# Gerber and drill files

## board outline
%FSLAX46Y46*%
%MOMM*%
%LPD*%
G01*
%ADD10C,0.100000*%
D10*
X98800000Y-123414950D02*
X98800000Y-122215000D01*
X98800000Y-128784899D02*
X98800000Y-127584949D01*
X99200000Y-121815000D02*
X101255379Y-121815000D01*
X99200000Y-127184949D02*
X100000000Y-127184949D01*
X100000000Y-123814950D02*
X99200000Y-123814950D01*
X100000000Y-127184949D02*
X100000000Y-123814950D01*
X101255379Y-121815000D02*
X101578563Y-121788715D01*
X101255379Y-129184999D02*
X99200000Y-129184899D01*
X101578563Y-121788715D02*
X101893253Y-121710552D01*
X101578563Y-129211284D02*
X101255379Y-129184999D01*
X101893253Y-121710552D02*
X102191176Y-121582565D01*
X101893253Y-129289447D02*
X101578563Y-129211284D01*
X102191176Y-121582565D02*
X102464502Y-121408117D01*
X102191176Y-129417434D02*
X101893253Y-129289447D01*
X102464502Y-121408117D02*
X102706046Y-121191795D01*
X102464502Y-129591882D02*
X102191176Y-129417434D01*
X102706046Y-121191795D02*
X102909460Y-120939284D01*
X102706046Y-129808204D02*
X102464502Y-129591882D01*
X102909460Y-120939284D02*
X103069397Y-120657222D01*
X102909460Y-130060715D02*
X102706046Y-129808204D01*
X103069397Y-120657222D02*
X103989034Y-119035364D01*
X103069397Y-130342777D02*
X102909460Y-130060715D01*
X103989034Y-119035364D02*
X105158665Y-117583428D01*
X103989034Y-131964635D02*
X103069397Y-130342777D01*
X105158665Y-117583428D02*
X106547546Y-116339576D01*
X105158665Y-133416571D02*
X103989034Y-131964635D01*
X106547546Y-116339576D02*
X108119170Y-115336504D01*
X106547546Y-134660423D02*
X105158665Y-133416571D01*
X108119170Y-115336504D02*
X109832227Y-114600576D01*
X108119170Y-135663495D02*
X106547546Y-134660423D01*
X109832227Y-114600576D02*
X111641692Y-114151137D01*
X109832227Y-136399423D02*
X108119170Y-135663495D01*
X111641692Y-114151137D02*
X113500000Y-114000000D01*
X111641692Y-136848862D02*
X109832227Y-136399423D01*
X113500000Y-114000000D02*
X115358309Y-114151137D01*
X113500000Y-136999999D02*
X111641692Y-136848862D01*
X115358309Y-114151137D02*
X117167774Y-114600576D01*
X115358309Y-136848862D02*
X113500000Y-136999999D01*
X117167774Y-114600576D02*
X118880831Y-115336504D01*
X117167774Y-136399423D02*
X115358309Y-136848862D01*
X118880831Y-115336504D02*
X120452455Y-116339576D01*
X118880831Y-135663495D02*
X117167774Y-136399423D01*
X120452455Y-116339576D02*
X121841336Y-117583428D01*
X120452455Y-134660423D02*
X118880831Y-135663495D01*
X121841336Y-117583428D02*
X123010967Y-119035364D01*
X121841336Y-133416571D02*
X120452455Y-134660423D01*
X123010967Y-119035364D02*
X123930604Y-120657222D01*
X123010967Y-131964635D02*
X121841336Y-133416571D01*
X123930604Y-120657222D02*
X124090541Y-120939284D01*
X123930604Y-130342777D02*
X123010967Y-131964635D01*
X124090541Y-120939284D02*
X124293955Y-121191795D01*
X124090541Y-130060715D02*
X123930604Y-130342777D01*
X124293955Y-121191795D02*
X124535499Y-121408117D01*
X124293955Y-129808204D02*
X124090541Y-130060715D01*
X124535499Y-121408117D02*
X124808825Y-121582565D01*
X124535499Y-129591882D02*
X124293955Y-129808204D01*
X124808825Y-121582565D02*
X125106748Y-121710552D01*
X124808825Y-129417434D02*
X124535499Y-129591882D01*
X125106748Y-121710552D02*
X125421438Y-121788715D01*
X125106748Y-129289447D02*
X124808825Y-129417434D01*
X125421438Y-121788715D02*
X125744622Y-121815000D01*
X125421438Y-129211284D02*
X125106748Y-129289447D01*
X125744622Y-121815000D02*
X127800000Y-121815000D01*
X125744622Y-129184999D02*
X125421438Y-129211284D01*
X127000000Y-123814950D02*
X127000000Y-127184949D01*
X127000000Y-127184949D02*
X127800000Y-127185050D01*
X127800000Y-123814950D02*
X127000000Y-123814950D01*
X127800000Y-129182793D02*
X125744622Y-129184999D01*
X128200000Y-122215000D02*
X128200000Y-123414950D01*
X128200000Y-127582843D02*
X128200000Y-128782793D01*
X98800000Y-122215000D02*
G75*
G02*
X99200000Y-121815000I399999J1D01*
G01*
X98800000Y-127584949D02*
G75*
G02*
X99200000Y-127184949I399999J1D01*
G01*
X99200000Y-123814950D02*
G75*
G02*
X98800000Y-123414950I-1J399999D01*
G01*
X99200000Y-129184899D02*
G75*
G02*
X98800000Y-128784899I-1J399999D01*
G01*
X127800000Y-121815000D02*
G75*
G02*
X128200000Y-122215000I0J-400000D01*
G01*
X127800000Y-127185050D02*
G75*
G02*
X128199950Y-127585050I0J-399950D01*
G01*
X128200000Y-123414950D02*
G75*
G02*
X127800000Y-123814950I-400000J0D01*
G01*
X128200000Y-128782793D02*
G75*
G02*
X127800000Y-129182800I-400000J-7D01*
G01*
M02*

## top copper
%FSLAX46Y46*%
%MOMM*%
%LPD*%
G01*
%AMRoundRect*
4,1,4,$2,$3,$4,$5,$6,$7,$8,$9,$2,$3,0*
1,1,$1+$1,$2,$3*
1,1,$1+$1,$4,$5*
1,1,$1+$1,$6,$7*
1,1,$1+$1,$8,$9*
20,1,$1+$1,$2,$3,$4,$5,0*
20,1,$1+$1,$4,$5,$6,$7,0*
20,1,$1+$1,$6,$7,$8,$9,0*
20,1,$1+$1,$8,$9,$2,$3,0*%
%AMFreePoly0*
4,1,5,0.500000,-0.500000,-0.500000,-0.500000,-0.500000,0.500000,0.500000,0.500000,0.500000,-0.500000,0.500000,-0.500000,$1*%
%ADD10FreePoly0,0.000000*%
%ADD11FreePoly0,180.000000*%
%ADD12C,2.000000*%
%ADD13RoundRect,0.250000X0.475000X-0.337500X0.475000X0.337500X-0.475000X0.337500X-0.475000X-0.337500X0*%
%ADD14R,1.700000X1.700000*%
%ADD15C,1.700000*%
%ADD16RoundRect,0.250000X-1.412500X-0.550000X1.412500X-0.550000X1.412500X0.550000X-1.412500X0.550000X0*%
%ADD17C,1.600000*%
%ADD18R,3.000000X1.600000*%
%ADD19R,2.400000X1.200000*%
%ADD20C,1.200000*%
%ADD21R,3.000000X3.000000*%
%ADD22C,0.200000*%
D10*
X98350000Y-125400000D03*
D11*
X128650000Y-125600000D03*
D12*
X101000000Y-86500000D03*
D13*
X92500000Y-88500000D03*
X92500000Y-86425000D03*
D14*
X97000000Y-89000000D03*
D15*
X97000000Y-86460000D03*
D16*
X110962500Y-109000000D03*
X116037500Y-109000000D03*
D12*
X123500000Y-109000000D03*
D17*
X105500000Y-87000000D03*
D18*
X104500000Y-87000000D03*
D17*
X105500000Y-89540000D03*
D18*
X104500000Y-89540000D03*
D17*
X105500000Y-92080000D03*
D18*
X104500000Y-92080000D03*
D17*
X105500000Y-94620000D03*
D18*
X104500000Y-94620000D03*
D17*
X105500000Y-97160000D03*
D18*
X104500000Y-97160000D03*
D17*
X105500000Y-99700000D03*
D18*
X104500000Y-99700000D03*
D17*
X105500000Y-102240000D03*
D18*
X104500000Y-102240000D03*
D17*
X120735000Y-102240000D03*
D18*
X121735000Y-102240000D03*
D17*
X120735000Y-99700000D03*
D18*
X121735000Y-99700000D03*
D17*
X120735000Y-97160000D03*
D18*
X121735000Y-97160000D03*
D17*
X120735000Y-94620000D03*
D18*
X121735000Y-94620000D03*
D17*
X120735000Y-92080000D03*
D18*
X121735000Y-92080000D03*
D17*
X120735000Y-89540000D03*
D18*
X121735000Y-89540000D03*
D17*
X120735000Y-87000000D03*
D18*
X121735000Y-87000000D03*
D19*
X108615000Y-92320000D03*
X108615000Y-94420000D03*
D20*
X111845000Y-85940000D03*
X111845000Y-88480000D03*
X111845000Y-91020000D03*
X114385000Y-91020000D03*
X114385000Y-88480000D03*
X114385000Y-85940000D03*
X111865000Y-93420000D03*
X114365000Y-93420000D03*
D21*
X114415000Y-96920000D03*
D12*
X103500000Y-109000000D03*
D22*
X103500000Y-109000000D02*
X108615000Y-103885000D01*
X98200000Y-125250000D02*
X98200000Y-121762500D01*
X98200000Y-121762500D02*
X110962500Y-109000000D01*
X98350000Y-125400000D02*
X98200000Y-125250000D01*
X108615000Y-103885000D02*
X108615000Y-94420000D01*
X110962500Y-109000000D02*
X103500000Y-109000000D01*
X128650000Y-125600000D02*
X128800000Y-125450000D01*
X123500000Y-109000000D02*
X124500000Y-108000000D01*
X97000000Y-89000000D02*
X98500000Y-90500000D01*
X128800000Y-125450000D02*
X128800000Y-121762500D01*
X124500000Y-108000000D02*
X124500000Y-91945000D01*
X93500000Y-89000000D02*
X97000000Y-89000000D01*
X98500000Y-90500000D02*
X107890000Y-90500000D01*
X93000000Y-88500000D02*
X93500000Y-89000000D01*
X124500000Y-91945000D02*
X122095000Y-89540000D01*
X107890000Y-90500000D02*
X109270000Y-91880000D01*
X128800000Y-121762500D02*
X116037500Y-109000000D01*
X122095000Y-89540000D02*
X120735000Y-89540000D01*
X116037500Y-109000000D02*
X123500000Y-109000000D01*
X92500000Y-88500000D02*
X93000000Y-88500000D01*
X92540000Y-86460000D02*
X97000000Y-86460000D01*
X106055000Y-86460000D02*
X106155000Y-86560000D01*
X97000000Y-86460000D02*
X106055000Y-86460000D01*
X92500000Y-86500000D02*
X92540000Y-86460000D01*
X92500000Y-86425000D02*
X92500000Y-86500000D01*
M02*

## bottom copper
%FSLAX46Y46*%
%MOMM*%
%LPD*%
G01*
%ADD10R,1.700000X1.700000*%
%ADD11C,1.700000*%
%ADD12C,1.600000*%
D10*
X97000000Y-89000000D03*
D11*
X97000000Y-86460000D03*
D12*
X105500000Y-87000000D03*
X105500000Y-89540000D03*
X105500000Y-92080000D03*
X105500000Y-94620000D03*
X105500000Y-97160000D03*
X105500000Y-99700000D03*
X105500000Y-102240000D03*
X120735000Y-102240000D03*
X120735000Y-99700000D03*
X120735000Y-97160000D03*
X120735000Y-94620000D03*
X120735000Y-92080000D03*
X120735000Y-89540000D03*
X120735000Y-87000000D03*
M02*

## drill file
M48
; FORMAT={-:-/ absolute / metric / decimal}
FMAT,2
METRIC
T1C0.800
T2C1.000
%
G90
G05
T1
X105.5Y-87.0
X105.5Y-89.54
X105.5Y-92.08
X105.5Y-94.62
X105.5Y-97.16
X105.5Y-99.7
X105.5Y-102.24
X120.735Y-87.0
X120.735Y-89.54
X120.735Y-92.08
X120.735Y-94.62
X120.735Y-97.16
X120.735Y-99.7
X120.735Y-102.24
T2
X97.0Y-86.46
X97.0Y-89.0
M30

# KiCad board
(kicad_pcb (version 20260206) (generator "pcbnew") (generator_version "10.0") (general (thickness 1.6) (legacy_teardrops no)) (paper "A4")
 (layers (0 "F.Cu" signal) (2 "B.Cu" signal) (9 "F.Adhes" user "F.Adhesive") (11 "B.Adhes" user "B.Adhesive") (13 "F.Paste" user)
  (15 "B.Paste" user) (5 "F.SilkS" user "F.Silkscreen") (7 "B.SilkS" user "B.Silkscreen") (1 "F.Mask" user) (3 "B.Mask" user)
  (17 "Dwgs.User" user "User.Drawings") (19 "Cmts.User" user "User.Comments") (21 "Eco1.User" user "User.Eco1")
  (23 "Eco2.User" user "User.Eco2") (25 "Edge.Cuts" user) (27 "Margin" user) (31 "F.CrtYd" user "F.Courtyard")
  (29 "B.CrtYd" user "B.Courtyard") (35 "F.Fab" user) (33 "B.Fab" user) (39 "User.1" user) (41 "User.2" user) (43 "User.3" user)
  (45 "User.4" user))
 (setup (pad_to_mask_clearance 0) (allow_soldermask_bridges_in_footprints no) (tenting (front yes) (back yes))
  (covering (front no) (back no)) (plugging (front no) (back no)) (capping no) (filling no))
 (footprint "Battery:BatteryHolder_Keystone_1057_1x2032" (layer "F.Cu") (at 113.5 125.5)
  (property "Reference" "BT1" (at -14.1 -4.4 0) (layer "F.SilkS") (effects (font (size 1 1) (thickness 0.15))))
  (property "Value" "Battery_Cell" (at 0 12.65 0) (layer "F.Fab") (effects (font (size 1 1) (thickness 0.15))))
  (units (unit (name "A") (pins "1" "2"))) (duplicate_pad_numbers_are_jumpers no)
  (fp_line (start -14.7 -2.08505) (end -14.7 -3.285) (stroke (width 0.1) (type solid)) (layer "Edge.Cuts"))
  (fp_line (start -14.7 3.284899) (end -14.7 2.084949) (stroke (width 0.1) (type solid)) (layer "Edge.Cuts"))
  (fp_line (start -14.3 -3.685) (end -12.244621 -3.685) (stroke (width 0.1) (type solid)) (layer "Edge.Cuts"))
  (fp_line (start -14.3 1.684949) (end -13.5 1.684949) (stroke (width 0.1) (type solid)) (layer "Edge.Cuts"))
  (fp_line (start -13.5 -1.68505) (end -14.3 -1.68505) (stroke (width 0.1) (type solid)) (layer "Edge.Cuts"))
  (fp_line (start -13.5 1.684949) (end -13.5 -1.68505) (stroke (width 0.1) (type solid)) (layer "Edge.Cuts"))
  (fp_line (start -12.244621 -3.685) (end -11.921437 -3.711285) (stroke (width 0.1) (type solid)) (layer "Edge.Cuts"))
  (fp_line (start -12.244621 3.684999) (end -14.3 3.684899) (stroke (width 0.1) (type solid)) (layer "Edge.Cuts"))
  (fp_line (start -11.921437 -3.711285) (end -11.606747 -3.789448) (stroke (width 0.1) (type solid)) (layer "Edge.Cuts"))
  (fp_line (start -11.921437 3.711284) (end -12.244621 3.684999) (stroke (width 0.1) (type solid)) (layer "Edge.Cuts"))
  (fp_line (start -11.606747 -3.789448) (end -11.308824 -3.917435) (stroke (width 0.1) (type solid)) (layer "Edge.Cuts"))
  (fp_line (start -11.606747 3.789447) (end -11.921437 3.711284) (stroke (width 0.1) (type solid)) (layer "Edge.Cuts"))
  (fp_line (start -11.308824 -3.917435) (end -11.035498 -4.091883) (stroke (width 0.1) (type solid)) (layer "Edge.Cuts"))
  (fp_line (start -11.308824 3.917434) (end -11.606747 3.789447) (stroke (width 0.1) (type solid)) (layer "Edge.Cuts"))
  (fp_line (start -11.035498 -4.091883) (end -10.793954 -4.308205) (stroke (width 0.1) (type solid)) (layer "Edge.Cuts"))
  (fp_line (start -11.035498 4.091882) (end -11.308824 3.917434) (stroke (width 0.1) (type solid)) (layer "Edge.Cuts"))
  (fp_line (start -10.793954 -4.308205) (end -10.59054 -4.560716) (stroke (width 0.1) (type solid)) (layer "Edge.Cuts"))
  (fp_line (start -10.793954 4.308204) (end -11.035498 4.091882) (stroke (width 0.1) (type solid)) (layer "Edge.Cuts"))
  (fp_line (start -10.59054 -4.560716) (end -10.430603 -4.842778) (stroke (width 0.1) (type solid)) (layer "Edge.Cuts"))
  (fp_line (start -10.59054 4.560715) (end -10.793954 4.308204) (stroke (width 0.1) (type solid)) (layer "Edge.Cuts"))
  (fp_line (start -10.430603 -4.842778) (end -9.510966 -6.464636) (stroke (width 0.1) (type solid)) (layer "Edge.Cuts"))
  (fp_line (start -10.430603 4.842777) (end -10.59054 4.560715) (stroke (width 0.1) (type solid)) (layer "Edge.Cuts"))
  (fp_line (start -9.510966 -6.464636) (end -8.341335 -7.916572) (stroke (width 0.1) (type solid)) (layer "Edge.Cuts"))
  (fp_line (start -9.510966 6.464635) (end -10.430603 4.842777) (stroke (width 0.1) (type solid)) (layer "Edge.Cuts"))
  (fp_line (start -8.341335 -7.916572) (end -6.952454 -9.160424) (stroke (width 0.1) (type solid)) (layer "Edge.Cuts"))
  (fp_line (start -8.341335 7.916571) (end -9.510966 6.464635) (stroke (width 0.1) (type solid)) (layer "Edge.Cuts"))
  (fp_line (start -6.952454 -9.160424) (end -5.38083 -10.163496) (stroke (width 0.1) (type solid)) (layer "Edge.Cuts"))
  (fp_line (start -6.952454 9.160423) (end -8.341335 7.916571) (stroke (width 0.1) (type solid)) (layer "Edge.Cuts"))
  (fp_line (start -5.38083 -10.163496) (end -3.667773 -10.899424) (stroke (width 0.1) (type solid)) (layer "Edge.Cuts"))
  (fp_line (start -5.38083 10.163495) (end -6.952454 9.160423) (stroke (width 0.1) (type solid)) (layer "Edge.Cuts"))
  (fp_line (start -3.667773 -10.899424) (end -1.858308 -11.348863) (stroke (width 0.1) (type solid)) (layer "Edge.Cuts"))
  (fp_line (start -3.667773 10.899423) (end -5.38083 10.163495) (stroke (width 0.1) (type solid)) (layer "Edge.Cuts"))
  (fp_line (start -1.858308 -11.348863) (end 0 -11.5) (stroke (width 0.1) (type solid)) (layer "Edge.Cuts"))
  (fp_line (start -1.858308 11.348862) (end -3.667773 10.899423) (stroke (width 0.1) (type solid)) (layer "Edge.Cuts"))
  (fp_line (start 0 -11.5) (end 1.858309 -11.348863) (stroke (width 0.1) (type solid)) (layer "Edge.Cuts"))
  (fp_line (start 0 11.499999) (end -1.858308 11.348862) (stroke (width 0.1) (type solid)) (layer "Edge.Cuts"))
  (fp_line (start 1.858309 -11.348863) (end 3.667774 -10.899424) (stroke (width 0.1) (type solid)) (layer "Edge.Cuts"))
  (fp_line (start 1.858309 11.348862) (end 0 11.499999) (stroke (width 0.1) (type solid)) (layer "Edge.Cuts"))
  (fp_line (start 3.667774 -10.899424) (end 5.380831 -10.163496) (stroke (width 0.1) (type solid)) (layer "Edge.Cuts"))
  (fp_line (start 3.667774 10.899423) (end 1.858309 11.348862) (stroke (width 0.1) (type solid)) (layer "Edge.Cuts"))
  (fp_line (start 5.380831 -10.163496) (end 6.952455 -9.160424) (stroke (width 0.1) (type solid)) (layer "Edge.Cuts"))
  (fp_line (start 5.380831 10.163495) (end 3.667774 10.899423) (stroke (width 0.1) (type solid)) (layer "Edge.Cuts"))
  (fp_line (start 6.952455 -9.160424) (end 8.341336 -7.916572) (stroke (width 0.1) (type solid)) (layer "Edge.Cuts"))
  (fp_line (start 6.952455 9.160423) (end 5.380831 10.163495) (stroke (width 0.1) (type solid)) (layer "Edge.Cuts"))
  (fp_line (start 8.341336 -7.916572) (end 9.510967 -6.464636) (stroke (width 0.1) (type solid)) (layer "Edge.Cuts"))
  (fp_line (start 8.341336 7.916571) (end 6.952455 9.160423) (stroke (width 0.1) (type solid)) (layer "Edge.Cuts"))
  (fp_line (start 9.510967 -6.464636) (end 10.430604 -4.842778) (stroke (width 0.1) (type solid)) (layer "Edge.Cuts"))
  (fp_line (start 9.510967 6.464635) (end 8.341336 7.916571) (stroke (width 0.1) (type solid)) (layer "Edge.Cuts"))
  (fp_line (start 10.430604 -4.842778) (end 10.590541 -4.560716) (stroke (width 0.1) (type solid)) (layer "Edge.Cuts"))
  (fp_line (start 10.430604 4.842777) (end 9.510967 6.464635) (stroke (width 0.1) (type solid)) (layer "Edge.Cuts"))
  (fp_line (start 10.590541 -4.560716) (end 10.793955 -4.308205) (stroke (width 0.1) (type solid)) (layer "Edge.Cuts"))
  (fp_line (start 10.590541 4.560715) (end 10.430604 4.842777) (stroke (width 0.1) (type solid)) (layer "Edge.Cuts"))
  (fp_line (start 10.793955 -4.308205) (end 11.035499 -4.091883) (stroke (width 0.1) (type solid)) (layer "Edge.Cuts"))
  (fp_line (start 10.793955 4.308204) (end 10.590541 4.560715) (stroke (width 0.1) (type solid)) (layer "Edge.Cuts"))
  (fp_line (start 11.035499 -4.091883) (end 11.308825 -3.917435) (stroke (width 0.1) (type solid)) (layer "Edge.Cuts"))
  (fp_line (start 11.035499 4.091882) (end 10.793955 4.308204) (stroke (width 0.1) (type solid)) (layer "Edge.Cuts"))
  (fp_line (start 11.308825 -3.917435) (end 11.606748 -3.789448) (stroke (width 0.1) (type solid)) (layer "Edge.Cuts"))
  (fp_line (start 11.308825 3.917434) (end 11.035499 4.091882) (stroke (width 0.1) (type solid)) (layer "Edge.Cuts"))
  (fp_line (start 11.606748 -3.789448) (end 11.921438 -3.711285) (stroke (width 0.1) (type solid)) (layer "Edge.Cuts"))
  (fp_line (start 11.606748 3.789447) (end 11.308825 3.917434) (stroke (width 0.1) (type solid)) (layer "Edge.Cuts"))
  (fp_line (start 11.921438 -3.711285) (end 12.244622 -3.685) (stroke (width 0.1) (type solid)) (layer "Edge.Cuts"))
  (fp_line (start 11.921438 3.711284) (end 11.606748 3.789447) (stroke (width 0.1) (type solid)) (layer "Edge.Cuts"))
  (fp_line (start 12.244622 -3.685) (end 14.3 -3.685) (stroke (width 0.1) (type solid)) (layer "Edge.Cuts"))
  (fp_line (start 12.244622 3.684999) (end 11.921438 3.711284) (stroke (width 0.1) (type solid)) (layer "Edge.Cuts"))
  (fp_line (start 13.5 -1.68505) (end 13.5 1.684949) (stroke (width 0.1) (type solid)) (layer "Edge.Cuts"))
  (fp_line (start 13.5 1.684949) (end 14.3 1.68505) (stroke (width 0.1) (type solid)) (layer "Edge.Cuts"))
  (fp_line (start 14.3 -1.68505) (end 13.5 -1.68505) (stroke (width 0.1) (type solid)) (layer "Edge.Cuts"))
  (fp_line (start 14.3 3.682793) (end 12.244622 3.684999) (stroke (width 0.1) (type solid)) (layer "Edge.Cuts"))
  (fp_line (start 14.7 -3.285) (end 14.7 -2.08505) (stroke (width 0.1) (type solid)) (layer "Edge.Cuts"))
  (fp_line (start 14.7 2.082843) (end 14.7 3.282793) (stroke (width 0.1) (type solid)) (layer "Edge.Cuts"))
  (fp_arc (start -14.7 -3.285) (mid -14.582843 -3.567843) (end -14.3 -3.685) (stroke (width 0.1) (type solid)) (layer "Edge.Cuts"))
  (fp_arc (start -14.7 2.084949) (mid -14.582843 1.802106) (end -14.3 1.684949) (stroke (width 0.1) (type solid)) (layer "Edge.Cuts"))
  (fp_arc (start -14.3 -1.68505) (mid -14.582843 -1.802207) (end -14.7 -2.08505) (stroke (width 0.1) (type solid)) (layer "Edge.Cuts"))
  (fp_arc (start -14.3 3.684899) (mid -14.582843 3.567742) (end -14.7 3.284899) (stroke (width 0.1) (type solid)) (layer "Edge.Cuts"))
  (fp_arc (start 14.3 -3.685) (mid 14.582843 -3.567843) (end 14.7 -3.285) (stroke (width 0.1) (type solid)) (layer "Edge.Cuts"))
  (fp_arc (start 14.3 1.68505) (mid 14.582843 1.802207) (end 14.7 2.08505) (stroke (width 0.1) (type solid)) (layer "Edge.Cuts"))
  (fp_arc (start 14.7 -2.08505) (mid 14.582843 -1.802207) (end 14.3 -1.68505) (stroke (width 0.1) (type solid)) (layer "Edge.Cuts"))
  (fp_arc (start 14.7 3.282793) (mid 14.582843 3.565636) (end 14.3 3.682793) (stroke (width 0.1) (type solid)) (layer "Edge.Cuts"))
  (pad "1" smd custom (at -15.15 -0.1) (size 1 1) (layers "F.Cu" "F.Mask" "F.Paste") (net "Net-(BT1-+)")
   (options (clearance outline) (anchor rect)) (primitives))
  (pad "2" smd custom (at 15.15 0.1 180) (size 1 1) (layers "F.Cu" "F.Mask" "F.Paste") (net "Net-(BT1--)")
   (options (clearance outline) (anchor rect)) (primitives)))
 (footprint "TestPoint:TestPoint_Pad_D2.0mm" (layer "F.Cu") (at 101 86.5)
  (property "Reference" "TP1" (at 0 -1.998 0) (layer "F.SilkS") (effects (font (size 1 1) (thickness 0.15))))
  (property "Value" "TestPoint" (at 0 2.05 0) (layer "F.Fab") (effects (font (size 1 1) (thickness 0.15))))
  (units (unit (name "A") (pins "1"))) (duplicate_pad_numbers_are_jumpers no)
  (pad "1" smd circle (at 0 0) (size 2 2) (layers "F.Cu" "F.Mask") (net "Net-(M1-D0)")))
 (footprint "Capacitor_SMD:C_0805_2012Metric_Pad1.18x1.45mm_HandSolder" (layer "F.Cu") (at 92.5 87.4625 90)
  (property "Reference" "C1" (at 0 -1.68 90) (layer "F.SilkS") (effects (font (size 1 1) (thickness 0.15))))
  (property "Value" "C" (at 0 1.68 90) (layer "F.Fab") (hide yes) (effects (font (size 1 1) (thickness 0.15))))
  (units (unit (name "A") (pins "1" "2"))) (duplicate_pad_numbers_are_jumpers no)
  (pad "1" smd roundrect (at -1.0375 0 90) (size 1.175 1.45) (layers "F.Cu" "F.Mask" "F.Paste") (roundrect_rratio 0.212766)
   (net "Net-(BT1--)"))
  (pad "2" smd roundrect (at 1.0375 0 90) (size 1.175 1.45) (layers "F.Cu" "F.Mask" "F.Paste") (roundrect_rratio 0.212766)
   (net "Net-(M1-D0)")))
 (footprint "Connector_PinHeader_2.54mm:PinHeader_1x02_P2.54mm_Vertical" (layer "F.Cu") (at 97 89 180)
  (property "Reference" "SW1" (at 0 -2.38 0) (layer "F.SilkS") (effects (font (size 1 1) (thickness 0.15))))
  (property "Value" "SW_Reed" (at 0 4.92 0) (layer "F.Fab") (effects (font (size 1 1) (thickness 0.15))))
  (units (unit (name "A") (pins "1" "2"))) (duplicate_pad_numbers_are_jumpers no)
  (pad "1" thru_hole rect (at 0 0 180) (size 1.7 1.7) (drill 1) (layers "*.Cu" "*.Mask") (remove_unused_layers no) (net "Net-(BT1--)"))
  (pad "2" thru_hole circle (at 0 2.54 180) (size 1.7 1.7) (drill 1) (layers "*.Cu" "*.Mask") (remove_unused_layers no) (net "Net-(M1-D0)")))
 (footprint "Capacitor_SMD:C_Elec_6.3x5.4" (layer "F.Cu") (at 113.5 109)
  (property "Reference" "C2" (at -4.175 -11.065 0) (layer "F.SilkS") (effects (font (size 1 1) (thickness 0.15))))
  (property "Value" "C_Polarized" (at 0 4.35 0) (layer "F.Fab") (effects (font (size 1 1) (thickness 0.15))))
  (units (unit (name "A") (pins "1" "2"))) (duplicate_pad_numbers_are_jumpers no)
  (pad "1" smd roundrect (at -2.5375 0) (size 3.325 1.6) (layers "F.Cu" "F.Mask" "F.Paste") (roundrect_rratio 0.15625) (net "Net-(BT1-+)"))
  (pad "2" smd roundrect (at 2.5375 0) (size 3.325 1.6) (layers "F.Cu" "F.Mask" "F.Paste") (roundrect_rratio 0.15625) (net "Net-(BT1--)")))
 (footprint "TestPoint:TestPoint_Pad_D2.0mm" (layer "F.Cu") (at 123.5 109)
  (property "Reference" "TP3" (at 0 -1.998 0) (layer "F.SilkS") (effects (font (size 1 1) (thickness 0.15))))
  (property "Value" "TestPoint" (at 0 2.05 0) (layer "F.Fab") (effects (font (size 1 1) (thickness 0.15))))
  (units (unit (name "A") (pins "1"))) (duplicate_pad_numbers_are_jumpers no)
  (pad "1" smd circle (at 0 0) (size 2 2) (layers "F.Cu" "F.Mask") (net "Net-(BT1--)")))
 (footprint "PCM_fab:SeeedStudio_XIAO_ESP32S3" (layer "F.Cu") (at 113.115 94.62)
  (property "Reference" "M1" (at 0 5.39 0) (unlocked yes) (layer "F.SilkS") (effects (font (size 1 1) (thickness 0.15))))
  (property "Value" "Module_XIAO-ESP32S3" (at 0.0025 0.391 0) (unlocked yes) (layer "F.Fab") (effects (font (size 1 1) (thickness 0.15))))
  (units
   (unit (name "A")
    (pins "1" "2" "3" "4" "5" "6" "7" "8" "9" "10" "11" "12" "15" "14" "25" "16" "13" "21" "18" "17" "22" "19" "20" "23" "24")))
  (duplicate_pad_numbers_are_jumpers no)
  (pad "1" thru_hole circle (at -7.615 -7.62) (size 1.6 1.6) (drill 0.8) (layers "*.Cu" "*.Mask") (remove_unused_layers no)
   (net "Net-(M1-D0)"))
  (pad "1" smd rect (at -7.615 -7.62) (size 3 1.6) (drill (offset -1 0)) (layers "F.Cu" "F.Mask" "F.Paste") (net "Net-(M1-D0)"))
  (pad "2" thru_hole circle (at -7.615 -5.08) (size 1.6 1.6) (drill 0.8) (layers "*.Cu" "*.Mask") (remove_unused_layers no)
   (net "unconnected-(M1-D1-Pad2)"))
  (pad "2" smd rect (at -7.615 -5.08) (size 3 1.6) (drill (offset -1 0)) (layers "F.Cu" "F.Mask" "F.Paste")
   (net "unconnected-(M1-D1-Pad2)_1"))
  (pad "3" thru_hole circle (at -7.615 -2.54) (size 1.6 1.6) (drill 0.8) (layers "*.Cu" "*.Mask") (remove_unused_layers no)
   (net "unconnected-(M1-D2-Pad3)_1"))
  (pad "3" smd rect (at -7.615 -2.54) (size 3 1.6) (drill (offset -1 0)) (layers "F.Cu" "F.Mask" "F.Paste") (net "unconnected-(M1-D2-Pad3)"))
  (pad "4" thru_hole circle (at -7.615 0) (size 1.6 1.6) (drill 0.8) (layers "*.Cu" "*.Mask") (remove_unused_layers no)
   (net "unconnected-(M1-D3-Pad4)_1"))
  (pad "4" smd rect (at -7.615 0) (size 3 1.6) (drill (offset -1 0)) (layers "F.Cu" "F.Mask" "F.Paste") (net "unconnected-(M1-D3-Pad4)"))
  (pad "5" thru_hole circle (at -7.615 2.54) (size 1.6 1.6) (drill 0.8) (layers "*.Cu" "*.Mask") (remove_unused_layers no)
   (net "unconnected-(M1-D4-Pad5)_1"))
  (pad "5" smd rect (at -7.615 2.54) (size 3 1.6) (drill (offset -1 0)) (layers "F.Cu" "F.Mask" "F.Paste") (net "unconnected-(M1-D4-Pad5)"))
  (pad "6" thru_hole circle (at -7.615 5.08) (size 1.6 1.6) (drill 0.8) (layers "*.Cu" "*.Mask") (remove_unused_layers no)
   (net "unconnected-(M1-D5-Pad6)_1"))
  (pad "6" smd rect (at -7.615 5.08) (size 3 1.6) (drill (offset -1 0)) (layers "F.Cu" "F.Mask" "F.Paste") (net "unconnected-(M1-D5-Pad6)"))
  (pad "7" thru_hole circle (at -7.615 7.62) (size 1.6 1.6) (drill 0.8) (layers "*.Cu" "*.Mask") (remove_unused_layers no)
   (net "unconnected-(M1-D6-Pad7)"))
  (pad "7" smd rect (at -7.615 7.62) (size 3 1.6) (drill (offset -1 0)) (layers "F.Cu" "F.Mask" "F.Paste")
   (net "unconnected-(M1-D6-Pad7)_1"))
  (pad "8" thru_hole circle (at 7.62 7.62) (size 1.6 1.6) (drill 0.8) (layers "*.Cu" "*.Mask") (remove_unused_layers no)
   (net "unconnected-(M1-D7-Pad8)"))
  (pad "8" smd rect (at 7.62 7.62) (size 3 1.6) (drill (offset 1 0)) (layers "F.Cu" "F.Mask" "F.Paste") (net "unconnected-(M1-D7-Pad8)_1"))
  (pad "9" thru_hole circle (at 7.62 5.08) (size 1.6 1.6) (drill 0.8) (layers "*.Cu" "*.Mask") (remove_unused_layers no)
   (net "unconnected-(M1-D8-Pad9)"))
  (pad "9" smd rect (at 7.62 5.08) (size 3 1.6) (drill (offset 1 0)) (layers "F.Cu" "F.Mask" "F.Paste") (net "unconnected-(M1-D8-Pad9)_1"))
  (pad "10" thru_hole circle (at 7.62 2.54) (size 1.6 1.6) (drill 0.8) (layers "*.Cu" "*.Mask") (remove_unused_layers no)
   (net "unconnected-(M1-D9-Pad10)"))
  (pad "10" smd rect (at 7.62 2.54) (size 3 1.6) (drill (offset 1 0)) (layers "F.Cu" "F.Mask" "F.Paste") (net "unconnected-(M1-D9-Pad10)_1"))
  (pad "11" thru_hole circle (at 7.62 0) (size 1.6 1.6) (drill 0.8) (layers "*.Cu" "*.Mask") (remove_unused_layers no)
   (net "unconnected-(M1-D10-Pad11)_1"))
  (pad "11" smd rect (at 7.62 0) (size 3 1.6) (drill (offset 1 0)) (layers "F.Cu" "F.Mask" "F.Paste") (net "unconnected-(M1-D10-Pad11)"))
  (pad "12" thru_hole circle (at 7.62 -2.54) (size 1.6 1.6) (drill 0.8) (layers "*.Cu" "*.Mask") (remove_unused_layers no)
   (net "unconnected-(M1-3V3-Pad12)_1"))
  (pad "12" smd rect (at 7.62 -2.54) (size 3 1.6) (drill (offset 1 0)) (layers "F.Cu" "F.Mask" "F.Paste") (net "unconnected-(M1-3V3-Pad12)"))
  (pad "13" thru_hole circle (at 7.62 -5.08) (size 1.6 1.6) (drill 0.8) (layers "*.Cu" "*.Mask") (remove_unused_layers no)
   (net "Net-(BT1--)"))
  (pad "13" smd rect (at 7.62 -5.08) (size 3 1.6) (drill (offset 1 0)) (layers "F.Cu" "F.Mask" "F.Paste") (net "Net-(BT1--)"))
  (pad "14" thru_hole circle (at 7.62 -7.62) (size 1.6 1.6) (drill 0.8) (layers "*.Cu" "*.Mask") (remove_unused_layers no)
   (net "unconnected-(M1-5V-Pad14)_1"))
  (pad "14" smd rect (at 7.62 -7.62) (size 3 1.6) (drill (offset 1 0)) (layers "F.Cu" "F.Mask" "F.Paste") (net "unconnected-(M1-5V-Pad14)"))
  (pad "15" smd rect (at -4.5 -2.3) (size 2.4 1.2) (layers "F.Cu" "F.Mask" "F.Paste") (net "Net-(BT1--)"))
  (pad "16" smd rect (at -4.5 -0.2) (size 2.4 1.2) (layers "F.Cu" "F.Mask" "F.Paste") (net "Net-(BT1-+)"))
  (pad "17" smd circle (at -1.27 -8.68) (size 1.2 1.2) (layers "F.Cu" "F.Mask" "F.Paste") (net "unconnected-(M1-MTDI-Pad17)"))
  (pad "18" smd circle (at -1.27 -6.14) (size 1.2 1.2) (layers "F.Cu" "F.Mask" "F.Paste") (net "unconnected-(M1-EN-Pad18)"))
  (pad "19" smd circle (at -1.27 -3.6) (size 1.2 1.2) (layers "F.Cu" "F.Mask" "F.Paste") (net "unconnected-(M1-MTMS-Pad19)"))
  (pad "20" smd circle (at 1.27 -3.6) (size 1.2 1.2) (layers "F.Cu" "F.Mask" "F.Paste") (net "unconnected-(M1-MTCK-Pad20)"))
  (pad "21" smd circle (at 1.27 -6.14) (size 1.2 1.2) (layers "F.Cu" "F.Mask" "F.Paste") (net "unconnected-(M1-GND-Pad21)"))
  (pad "22" smd circle (at 1.27 -8.68) (size 1.2 1.2) (layers "F.Cu" "F.Mask" "F.Paste") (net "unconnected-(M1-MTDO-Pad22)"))
  (pad "23" smd circle (at -1.25 -1.2) (size 1.2 1.2) (layers "F.Cu" "F.Mask" "F.Paste") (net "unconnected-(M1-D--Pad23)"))
  (pad "24" smd circle (at 1.25 -1.2) (size 1.2 1.2) (layers "F.Cu" "F.Mask" "F.Paste") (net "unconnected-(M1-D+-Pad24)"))
  (pad "25" smd rect (at 1.3 2.3) (size 3 3) (layers "F.Cu" "F.Mask" "F.Paste") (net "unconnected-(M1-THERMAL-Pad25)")))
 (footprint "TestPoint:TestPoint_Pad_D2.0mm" (layer "F.Cu") (at 103.5 109)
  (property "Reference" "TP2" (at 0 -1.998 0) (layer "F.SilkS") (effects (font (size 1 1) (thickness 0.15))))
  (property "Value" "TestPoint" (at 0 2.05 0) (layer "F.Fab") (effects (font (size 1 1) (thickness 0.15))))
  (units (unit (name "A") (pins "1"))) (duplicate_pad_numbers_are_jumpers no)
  (pad "1" smd circle (at 0 0) (size 2 2) (layers "F.Cu" "F.Mask") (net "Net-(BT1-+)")))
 (segment (start 103.5 109) (end 108.615 103.885) (width 0.2) (layer "F.Cu") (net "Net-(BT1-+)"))
 (segment (start 98.2 125.25) (end 98.2 121.7625) (width 0.2) (layer "F.Cu") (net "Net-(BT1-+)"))
 (segment (start 98.2 121.7625) (end 110.9625 109) (width 0.2) (layer "F.Cu") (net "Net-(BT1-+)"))
 (segment (start 98.35 125.4) (end 98.2 125.25) (width 0.2) (layer "F.Cu") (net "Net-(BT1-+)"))
 (segment (start 108.615 103.885) (end 108.615 94.42) (width 0.2) (layer "F.Cu") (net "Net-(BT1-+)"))
 (segment (start 110.9625 109) (end 103.5 109) (width 0.2) (layer "F.Cu") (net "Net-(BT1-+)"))
 (segment (start 128.65 125.6) (end 128.8 125.45) (width 0.2) (layer "F.Cu") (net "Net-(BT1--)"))
 (segment (start 123.5 109) (end 124.5 108) (width 0.2) (layer "F.Cu") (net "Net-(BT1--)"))
 (segment (start 97 89) (end 98.5 90.5) (width 0.2) (layer "F.Cu") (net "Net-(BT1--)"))
 (segment (start 128.8 125.45) (end 128.8 121.7625) (width 0.2) (layer "F.Cu") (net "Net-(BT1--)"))
 (segment (start 124.5 108) (end 124.5 91.945) (width 0.2) (layer "F.Cu") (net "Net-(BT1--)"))
 (segment (start 93.5 89) (end 97 89) (width 0.2) (layer "F.Cu") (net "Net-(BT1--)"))
 (segment (start 98.5 90.5) (end 107.89 90.5) (width 0.2) (layer "F.Cu") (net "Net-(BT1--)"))
 (segment (start 93 88.5) (end 93.5 89) (width 0.2) (layer "F.Cu") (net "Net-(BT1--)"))
 (segment (start 124.5 91.945) (end 122.095 89.54) (width 0.2) (layer "F.Cu") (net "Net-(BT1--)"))
 (segment (start 107.89 90.5) (end 109.27 91.88) (width 0.2) (layer "F.Cu") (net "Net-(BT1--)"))
 (segment (start 128.8 121.7625) (end 116.0375 109) (width 0.2) (layer "F.Cu") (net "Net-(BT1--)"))
 (segment (start 122.095 89.54) (end 120.735 89.54) (width 0.2) (layer "F.Cu") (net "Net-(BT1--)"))
 (segment (start 116.0375 109) (end 123.5 109) (width 0.2) (layer "F.Cu") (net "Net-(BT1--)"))
 (segment (start 92.5 88.5) (end 93 88.5) (width 0.2) (layer "F.Cu") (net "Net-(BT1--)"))
 (segment (start 92.54 86.46) (end 97 86.46) (width 0.2) (layer "F.Cu") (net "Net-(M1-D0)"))
 (segment (start 106.055 86.46) (end 106.155 86.56) (width 0.2) (layer "F.Cu") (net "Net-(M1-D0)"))
 (segment (start 97 86.46) (end 106.055 86.46) (width 0.2) (layer "F.Cu") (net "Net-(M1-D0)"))
 (segment (start 92.5 86.5) (end 92.54 86.46) (width 0.2) (layer "F.Cu") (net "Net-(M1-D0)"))
 (segment (start 92.5 86.425) (end 92.5 86.5) (width 0.2) (layer "F.Cu") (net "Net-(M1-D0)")))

